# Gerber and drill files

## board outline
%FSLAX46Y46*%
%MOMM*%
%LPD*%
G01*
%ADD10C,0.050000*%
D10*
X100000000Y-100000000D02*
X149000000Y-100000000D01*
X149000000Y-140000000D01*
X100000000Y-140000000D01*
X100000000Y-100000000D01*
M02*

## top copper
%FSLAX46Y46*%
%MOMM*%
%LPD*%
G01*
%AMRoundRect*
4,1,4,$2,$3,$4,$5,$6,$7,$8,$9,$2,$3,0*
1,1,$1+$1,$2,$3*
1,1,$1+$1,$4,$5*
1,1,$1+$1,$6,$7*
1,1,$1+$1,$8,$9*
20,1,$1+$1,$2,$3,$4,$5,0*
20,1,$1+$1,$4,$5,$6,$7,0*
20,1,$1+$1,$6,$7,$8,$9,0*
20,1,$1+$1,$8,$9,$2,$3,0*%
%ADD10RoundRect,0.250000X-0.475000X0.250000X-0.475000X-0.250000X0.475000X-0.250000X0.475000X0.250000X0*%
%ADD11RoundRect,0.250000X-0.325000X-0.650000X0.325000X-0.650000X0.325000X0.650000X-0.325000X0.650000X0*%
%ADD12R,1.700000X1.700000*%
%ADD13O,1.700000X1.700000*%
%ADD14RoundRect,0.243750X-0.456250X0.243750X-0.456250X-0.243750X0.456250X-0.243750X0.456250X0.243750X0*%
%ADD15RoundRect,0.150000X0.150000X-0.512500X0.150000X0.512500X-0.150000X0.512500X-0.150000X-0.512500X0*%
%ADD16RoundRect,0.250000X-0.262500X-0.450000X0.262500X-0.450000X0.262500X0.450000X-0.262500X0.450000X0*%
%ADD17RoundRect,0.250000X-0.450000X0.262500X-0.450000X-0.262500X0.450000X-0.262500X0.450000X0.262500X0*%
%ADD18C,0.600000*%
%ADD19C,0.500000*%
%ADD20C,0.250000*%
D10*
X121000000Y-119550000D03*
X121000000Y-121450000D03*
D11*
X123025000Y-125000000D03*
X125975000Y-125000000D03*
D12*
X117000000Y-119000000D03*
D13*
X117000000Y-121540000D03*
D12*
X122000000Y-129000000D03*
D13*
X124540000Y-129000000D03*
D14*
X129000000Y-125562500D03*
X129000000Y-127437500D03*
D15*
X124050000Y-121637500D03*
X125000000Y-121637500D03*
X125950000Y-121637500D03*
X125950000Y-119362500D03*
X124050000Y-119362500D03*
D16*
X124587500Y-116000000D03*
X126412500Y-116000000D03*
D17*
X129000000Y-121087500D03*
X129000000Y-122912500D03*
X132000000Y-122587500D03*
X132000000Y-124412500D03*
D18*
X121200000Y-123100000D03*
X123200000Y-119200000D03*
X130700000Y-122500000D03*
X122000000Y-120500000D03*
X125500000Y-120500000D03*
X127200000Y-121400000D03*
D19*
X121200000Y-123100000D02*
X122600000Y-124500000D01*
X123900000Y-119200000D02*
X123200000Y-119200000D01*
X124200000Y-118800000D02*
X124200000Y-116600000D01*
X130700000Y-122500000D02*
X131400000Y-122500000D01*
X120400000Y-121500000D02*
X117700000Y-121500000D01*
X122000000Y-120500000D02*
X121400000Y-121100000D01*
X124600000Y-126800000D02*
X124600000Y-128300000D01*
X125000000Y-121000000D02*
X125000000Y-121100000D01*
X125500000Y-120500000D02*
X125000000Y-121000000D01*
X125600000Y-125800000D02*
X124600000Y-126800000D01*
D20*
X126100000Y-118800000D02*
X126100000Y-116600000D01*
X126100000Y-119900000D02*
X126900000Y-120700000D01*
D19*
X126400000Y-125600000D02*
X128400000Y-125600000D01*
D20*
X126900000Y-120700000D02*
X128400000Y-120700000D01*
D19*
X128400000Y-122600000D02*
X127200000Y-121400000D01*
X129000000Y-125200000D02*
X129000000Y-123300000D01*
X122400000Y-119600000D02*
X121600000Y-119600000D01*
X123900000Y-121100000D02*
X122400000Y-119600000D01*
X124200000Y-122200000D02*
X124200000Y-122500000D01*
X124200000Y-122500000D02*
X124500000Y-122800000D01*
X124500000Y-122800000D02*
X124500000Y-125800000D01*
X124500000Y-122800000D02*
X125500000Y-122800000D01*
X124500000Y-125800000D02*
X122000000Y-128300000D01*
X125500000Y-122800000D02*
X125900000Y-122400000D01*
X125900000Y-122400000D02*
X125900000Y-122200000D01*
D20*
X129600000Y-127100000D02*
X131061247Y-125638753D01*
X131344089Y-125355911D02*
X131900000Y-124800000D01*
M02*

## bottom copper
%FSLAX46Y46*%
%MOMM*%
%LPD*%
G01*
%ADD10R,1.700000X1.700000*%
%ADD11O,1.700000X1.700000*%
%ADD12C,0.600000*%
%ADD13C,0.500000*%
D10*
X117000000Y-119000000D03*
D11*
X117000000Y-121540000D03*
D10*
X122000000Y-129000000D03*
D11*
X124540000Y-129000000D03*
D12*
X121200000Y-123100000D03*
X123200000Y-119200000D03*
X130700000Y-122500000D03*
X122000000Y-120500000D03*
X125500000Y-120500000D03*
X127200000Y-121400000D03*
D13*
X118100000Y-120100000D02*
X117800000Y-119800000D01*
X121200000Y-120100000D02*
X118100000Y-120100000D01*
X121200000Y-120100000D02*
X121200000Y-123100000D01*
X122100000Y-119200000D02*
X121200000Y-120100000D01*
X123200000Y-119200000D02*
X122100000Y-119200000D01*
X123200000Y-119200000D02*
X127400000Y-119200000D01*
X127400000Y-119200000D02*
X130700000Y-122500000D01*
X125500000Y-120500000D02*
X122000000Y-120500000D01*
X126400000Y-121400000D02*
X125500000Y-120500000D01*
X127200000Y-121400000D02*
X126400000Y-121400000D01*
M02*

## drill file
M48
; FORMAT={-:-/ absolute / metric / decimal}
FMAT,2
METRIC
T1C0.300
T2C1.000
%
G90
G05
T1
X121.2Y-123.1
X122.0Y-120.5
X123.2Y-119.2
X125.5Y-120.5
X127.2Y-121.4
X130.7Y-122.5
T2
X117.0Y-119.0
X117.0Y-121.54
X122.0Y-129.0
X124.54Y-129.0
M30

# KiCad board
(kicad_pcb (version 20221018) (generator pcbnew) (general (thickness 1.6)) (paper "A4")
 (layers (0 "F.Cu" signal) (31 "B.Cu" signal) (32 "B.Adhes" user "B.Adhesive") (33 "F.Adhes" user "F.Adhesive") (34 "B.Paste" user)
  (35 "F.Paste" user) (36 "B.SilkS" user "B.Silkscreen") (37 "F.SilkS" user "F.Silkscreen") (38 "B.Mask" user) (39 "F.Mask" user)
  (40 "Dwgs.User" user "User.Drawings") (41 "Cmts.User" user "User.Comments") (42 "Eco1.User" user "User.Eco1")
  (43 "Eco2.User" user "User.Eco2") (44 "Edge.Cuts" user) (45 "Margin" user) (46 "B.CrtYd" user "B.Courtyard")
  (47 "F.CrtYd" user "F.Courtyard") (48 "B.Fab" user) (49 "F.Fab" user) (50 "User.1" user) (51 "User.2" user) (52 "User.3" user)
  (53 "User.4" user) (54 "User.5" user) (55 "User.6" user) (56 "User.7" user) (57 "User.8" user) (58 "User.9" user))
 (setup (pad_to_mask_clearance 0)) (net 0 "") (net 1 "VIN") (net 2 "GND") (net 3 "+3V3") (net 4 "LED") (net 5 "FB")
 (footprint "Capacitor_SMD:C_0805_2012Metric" (layer "F.Cu") (at 121 120.5 -90)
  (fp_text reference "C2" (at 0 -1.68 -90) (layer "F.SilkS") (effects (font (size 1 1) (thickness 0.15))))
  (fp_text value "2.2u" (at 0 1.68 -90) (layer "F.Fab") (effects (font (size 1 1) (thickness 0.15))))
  (pad "1" smd roundrect (at -0.95 0 270) (size 1 1.45) (layers "F.Cu" "F.Paste" "F.Mask") (roundrect_rratio 0.25) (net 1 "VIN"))
  (pad "2" smd roundrect (at 0.95 0 270) (size 1 1.45) (layers "F.Cu" "F.Paste" "F.Mask") (roundrect_rratio 0.25) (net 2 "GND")))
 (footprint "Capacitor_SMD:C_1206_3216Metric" (layer "F.Cu") (at 124.5 125)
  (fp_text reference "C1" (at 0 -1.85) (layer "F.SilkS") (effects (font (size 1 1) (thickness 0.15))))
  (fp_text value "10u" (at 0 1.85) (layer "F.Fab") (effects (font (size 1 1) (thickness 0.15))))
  (pad "1" smd roundrect (at -1.475 0) (size 1.15 1.8) (layers "F.Cu" "F.Paste" "F.Mask") (roundrect_rratio 0.217391) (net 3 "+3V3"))
  (pad "2" smd roundrect (at 1.475 0) (size 1.15 1.8) (layers "F.Cu" "F.Paste" "F.Mask") (roundrect_rratio 0.217391) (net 2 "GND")))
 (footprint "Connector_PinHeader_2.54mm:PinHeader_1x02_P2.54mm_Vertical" (layer "F.Cu") (at 117 119)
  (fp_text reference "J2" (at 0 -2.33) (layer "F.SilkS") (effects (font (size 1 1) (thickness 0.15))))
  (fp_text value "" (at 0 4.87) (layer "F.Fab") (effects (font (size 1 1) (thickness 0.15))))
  (pad "1" thru_hole rect (at 0 0) (size 1.7 1.7) (drill 1) (layers "*.Cu" "*.Mask") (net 3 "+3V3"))
  (pad "2" thru_hole oval (at 0 2.54) (size 1.7 1.7) (drill 1) (layers "*.Cu" "*.Mask") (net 2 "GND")))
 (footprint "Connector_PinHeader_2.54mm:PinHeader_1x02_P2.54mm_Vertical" (layer "F.Cu") (at 122 129 90)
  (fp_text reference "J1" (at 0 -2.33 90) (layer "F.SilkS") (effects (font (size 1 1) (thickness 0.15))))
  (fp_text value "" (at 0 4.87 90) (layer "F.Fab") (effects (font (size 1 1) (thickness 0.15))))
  (pad "1" thru_hole rect (at 0 0 90) (size 1.7 1.7) (drill 1) (layers "*.Cu" "*.Mask") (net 1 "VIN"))
  (pad "2" thru_hole oval (at 0 2.54 90) (size 1.7 1.7) (drill 1) (layers "*.Cu" "*.Mask") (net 2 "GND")))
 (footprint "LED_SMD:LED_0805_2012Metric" (layer "F.Cu") (at 129 126.5 -90)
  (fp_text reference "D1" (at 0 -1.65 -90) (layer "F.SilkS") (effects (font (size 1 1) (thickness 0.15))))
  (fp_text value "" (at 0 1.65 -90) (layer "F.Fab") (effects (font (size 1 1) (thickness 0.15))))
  (pad "1" smd roundrect (at -0.9375 0 270) (size 0.975 1.4) (layers "F.Cu" "F.Paste" "F.Mask") (roundrect_rratio 0.25) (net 2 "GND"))
  (pad "2" smd roundrect (at 0.9375 0 270) (size 0.975 1.4) (layers "F.Cu" "F.Paste" "F.Mask") (roundrect_rratio 0.25) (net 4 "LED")))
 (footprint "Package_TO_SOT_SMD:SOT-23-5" (layer "F.Cu") (at 125 120.5 90)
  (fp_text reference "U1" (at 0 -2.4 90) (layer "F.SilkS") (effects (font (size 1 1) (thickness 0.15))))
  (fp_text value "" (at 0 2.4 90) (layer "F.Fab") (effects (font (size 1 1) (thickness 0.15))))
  (pad "1" smd roundrect (at -1.1375 -0.95 90) (size 1.325 0.6) (layers "F.Cu" "F.Paste" "F.Mask") (roundrect_rratio 0.25) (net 1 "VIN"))
  (pad "2" smd roundrect (at -1.1375 0 90) (size 1.325 0.6) (layers "F.Cu" "F.Paste" "F.Mask") (roundrect_rratio 0.25) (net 2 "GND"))
  (pad "3" smd roundrect (at -1.1375 0.95 90) (size 1.325 0.6) (layers "F.Cu" "F.Paste" "F.Mask") (roundrect_rratio 0.25) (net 1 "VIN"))
  (pad "4" smd roundrect (at 1.1375 0.95 90) (size 1.325 0.6) (layers "F.Cu" "F.Paste" "F.Mask") (roundrect_rratio 0.25) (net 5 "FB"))
  (pad "5" smd roundrect (at 1.1375 -0.95 90) (size 1.325 0.6) (layers "F.Cu" "F.Paste" "F.Mask") (roundrect_rratio 0.25) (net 3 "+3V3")))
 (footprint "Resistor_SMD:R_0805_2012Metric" (layer "F.Cu") (at 125.5 116)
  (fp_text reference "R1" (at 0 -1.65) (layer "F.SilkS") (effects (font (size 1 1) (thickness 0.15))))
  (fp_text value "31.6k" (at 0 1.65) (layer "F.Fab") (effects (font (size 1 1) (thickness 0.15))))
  (pad "1" smd roundrect (at -0.9125 0) (size 1.025 1.4) (layers "F.Cu" "F.Paste" "F.Mask") (roundrect_rratio 0.243902) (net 3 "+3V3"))
  (pad "2" smd roundrect (at 0.9125 0) (size 1.025 1.4) (layers "F.Cu" "F.Paste" "F.Mask") (roundrect_rratio 0.243902) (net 5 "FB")))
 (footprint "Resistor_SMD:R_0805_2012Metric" (layer "F.Cu") (at 129 122 -90)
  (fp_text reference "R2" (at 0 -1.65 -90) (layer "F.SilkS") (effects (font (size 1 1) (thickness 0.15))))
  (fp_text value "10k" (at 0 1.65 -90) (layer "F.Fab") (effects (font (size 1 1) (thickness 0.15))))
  (pad "1" smd roundrect (at -0.9125 0 270) (size 1.025 1.4) (layers "F.Cu" "F.Paste" "F.Mask") (roundrect_rratio 0.243902) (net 5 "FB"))
  (pad "2" smd roundrect (at 0.9125 0 270) (size 1.025 1.4) (layers "F.Cu" "F.Paste" "F.Mask") (roundrect_rratio 0.243902) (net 2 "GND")))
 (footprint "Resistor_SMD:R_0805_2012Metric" (layer "F.Cu") (at 132 123.5 -90)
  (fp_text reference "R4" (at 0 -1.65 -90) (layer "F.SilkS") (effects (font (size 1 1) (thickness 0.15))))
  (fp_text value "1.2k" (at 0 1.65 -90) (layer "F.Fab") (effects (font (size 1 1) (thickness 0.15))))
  (pad "1" smd roundrect (at -0.9125 0 270) (size 1.025 1.4) (layers "F.Cu" "F.Paste" "F.Mask") (roundrect_rratio 0.243902) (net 3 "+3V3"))
  (pad "2" smd roundrect (at 0.9125 0 270) (size 1.025 1.4) (layers "F.Cu" "F.Paste" "F.Mask") (roundrect_rratio 0.243902) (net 4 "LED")))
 (gr_rect (start 100 100) (end 149 140) (stroke (width 0.05) (type default)) (fill none) (layer "Edge.Cuts"))
 (segment (start 121.2 123.1) (end 122.6 124.5) (width 0.5) (layer "F.Cu") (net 3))
 (segment (start 123.9 119.2) (end 123.2 119.2) (width 0.5) (layer "F.Cu") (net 3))
 (segment (start 124.2 118.8) (end 124.2 116.6) (width 0.5) (layer "F.Cu") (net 3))
 (segment (start 130.7 122.5) (end 131.4 122.5) (width 0.5) (layer "F.Cu") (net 3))
 (via (at 121.2 123.1) (size 0.6) (drill 0.3) (layers "F.Cu" "B.Cu") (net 3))
 (via (at 123.2 119.2) (size 0.6) (drill 0.3) (layers "F.Cu" "B.Cu") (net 3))
 (via (at 130.7 122.5) (size 0.6) (drill 0.3) (layers "F.Cu" "B.Cu") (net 3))
 (segment (start 118.1 120.1) (end 117.8 119.8) (width 0.5) (layer "B.Cu") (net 3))
 (segment (start 120.4 121.5) (end 117.7 121.5) (width 0.5) (layer "F.Cu") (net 2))
 (segment (start 121.2 120.1) (end 118.1 120.1) (width 0.5) (layer "B.Cu") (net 3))
 (segment (start 121.2 120.1) (end 121.2 123.1) (width 0.5) (layer "B.Cu") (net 3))
 (segment (start 122 120.5) (end 121.4 121.1) (width 0.5) (layer "F.Cu") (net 2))
 (segment (start 122.1 119.2) (end 121.2 120.1) (width 0.5) (layer "B.Cu") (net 3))
 (segment (start 123.2 119.2) (end 122.1 119.2) (width 0.5) (layer "B.Cu") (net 3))
 (segment (start 123.2 119.2) (end 127.4 119.2) (width 0.5) (layer "B.Cu") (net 3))
 (segment (start 124.6 126.8) (end 124.6 128.3) (width 0.5) (layer "F.Cu") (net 2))
 (segment (start 125 121) (end 125 121.1) (width 0.5) (layer "F.Cu") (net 2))
 (segment (start 125.5 120.5) (end 125 121) (width 0.5) (layer "F.Cu") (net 2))
 (segment (start 125.6 125.8) (end 124.6 126.8) (width 0.5) (layer "F.Cu") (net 2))
 (segment (start 126.1 118.8) (end 126.1 116.6) (width 0.25) (layer "F.Cu") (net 5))
 (segment (start 126.1 119.9) (end 126.9 120.7) (width 0.25) (layer "F.Cu") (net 5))
 (segment (start 126.4 125.6) (end 128.4 125.6) (width 0.5) (layer "F.Cu") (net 2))
 (segment (start 126.9 120.7) (end 128.4 120.7) (width 0.25) (layer "F.Cu") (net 5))
 (segment (start 127.4 119.2) (end 130.7 122.5) (width 0.5) (layer "B.Cu") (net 3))
 (segment (start 128.4 122.6) (end 127.2 121.4) (width 0.5) (layer "F.Cu") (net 2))
 (segment (start 129 125.2) (end 129 123.3) (width 0.5) (layer "F.Cu") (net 2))
 (via (at 122 120.5) (size 0.6) (drill 0.3) (layers "F.Cu" "B.Cu") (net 2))
 (via (at 125.5 120.5) (size 0.6) (drill 0.3) (layers "F.Cu" "B.Cu") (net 2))
 (via (at 127.2 121.4) (size 0.6) (drill 0.3) (layers "F.Cu" "B.Cu") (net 2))
 (segment (start 122.4 119.6) (end 121.6 119.6) (width 0.5) (layer "F.Cu") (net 1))
 (segment (start 123.9 121.1) (end 122.4 119.6) (width 0.5) (layer "F.Cu") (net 1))
 (segment (start 124.2 122.2) (end 124.2 122.5) (width 0.5) (layer "F.Cu") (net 1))
 (segment (start 124.2 122.5) (end 124.5 122.8) (width 0.5) (layer "F.Cu") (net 1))
 (segment (start 124.5 122.8) (end 124.5 125.8) (width 0.5) (layer "F.Cu") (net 1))
 (segment (start 124.5 122.8) (end 125.5 122.8) (width 0.5) (layer "F.Cu") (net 1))
 (segment (start 124.5 125.8) (end 122 128.3) (width 0.5) (layer "F.Cu") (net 1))
 (segment (start 125.5 120.5) (end 122 120.5) (width 0.5) (layer "B.Cu") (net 2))
 (segment (start 125.5 122.8) (end 125.9 122.4) (width 0.5) (layer "F.Cu") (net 1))
 (segment (start 125.9 122.4) (end 125.9 122.2) (width 0.5) (layer "F.Cu") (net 1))
 (segment (start 126.4 121.4) (end 125.5 120.5) (width 0.5) (layer "B.Cu") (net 2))
 (segment (start 127.2 121.4) (end 126.4 121.4) (width 0.5) (layer "B.Cu") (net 2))
 (segment (start 129.6 127.1) (end 131.061247 125.638753) (width 0.25) (layer "F.Cu") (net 4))
 (segment (start 131.344089 125.355911) (end 131.9 124.8) (width 0.25) (layer "F.Cu") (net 4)))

